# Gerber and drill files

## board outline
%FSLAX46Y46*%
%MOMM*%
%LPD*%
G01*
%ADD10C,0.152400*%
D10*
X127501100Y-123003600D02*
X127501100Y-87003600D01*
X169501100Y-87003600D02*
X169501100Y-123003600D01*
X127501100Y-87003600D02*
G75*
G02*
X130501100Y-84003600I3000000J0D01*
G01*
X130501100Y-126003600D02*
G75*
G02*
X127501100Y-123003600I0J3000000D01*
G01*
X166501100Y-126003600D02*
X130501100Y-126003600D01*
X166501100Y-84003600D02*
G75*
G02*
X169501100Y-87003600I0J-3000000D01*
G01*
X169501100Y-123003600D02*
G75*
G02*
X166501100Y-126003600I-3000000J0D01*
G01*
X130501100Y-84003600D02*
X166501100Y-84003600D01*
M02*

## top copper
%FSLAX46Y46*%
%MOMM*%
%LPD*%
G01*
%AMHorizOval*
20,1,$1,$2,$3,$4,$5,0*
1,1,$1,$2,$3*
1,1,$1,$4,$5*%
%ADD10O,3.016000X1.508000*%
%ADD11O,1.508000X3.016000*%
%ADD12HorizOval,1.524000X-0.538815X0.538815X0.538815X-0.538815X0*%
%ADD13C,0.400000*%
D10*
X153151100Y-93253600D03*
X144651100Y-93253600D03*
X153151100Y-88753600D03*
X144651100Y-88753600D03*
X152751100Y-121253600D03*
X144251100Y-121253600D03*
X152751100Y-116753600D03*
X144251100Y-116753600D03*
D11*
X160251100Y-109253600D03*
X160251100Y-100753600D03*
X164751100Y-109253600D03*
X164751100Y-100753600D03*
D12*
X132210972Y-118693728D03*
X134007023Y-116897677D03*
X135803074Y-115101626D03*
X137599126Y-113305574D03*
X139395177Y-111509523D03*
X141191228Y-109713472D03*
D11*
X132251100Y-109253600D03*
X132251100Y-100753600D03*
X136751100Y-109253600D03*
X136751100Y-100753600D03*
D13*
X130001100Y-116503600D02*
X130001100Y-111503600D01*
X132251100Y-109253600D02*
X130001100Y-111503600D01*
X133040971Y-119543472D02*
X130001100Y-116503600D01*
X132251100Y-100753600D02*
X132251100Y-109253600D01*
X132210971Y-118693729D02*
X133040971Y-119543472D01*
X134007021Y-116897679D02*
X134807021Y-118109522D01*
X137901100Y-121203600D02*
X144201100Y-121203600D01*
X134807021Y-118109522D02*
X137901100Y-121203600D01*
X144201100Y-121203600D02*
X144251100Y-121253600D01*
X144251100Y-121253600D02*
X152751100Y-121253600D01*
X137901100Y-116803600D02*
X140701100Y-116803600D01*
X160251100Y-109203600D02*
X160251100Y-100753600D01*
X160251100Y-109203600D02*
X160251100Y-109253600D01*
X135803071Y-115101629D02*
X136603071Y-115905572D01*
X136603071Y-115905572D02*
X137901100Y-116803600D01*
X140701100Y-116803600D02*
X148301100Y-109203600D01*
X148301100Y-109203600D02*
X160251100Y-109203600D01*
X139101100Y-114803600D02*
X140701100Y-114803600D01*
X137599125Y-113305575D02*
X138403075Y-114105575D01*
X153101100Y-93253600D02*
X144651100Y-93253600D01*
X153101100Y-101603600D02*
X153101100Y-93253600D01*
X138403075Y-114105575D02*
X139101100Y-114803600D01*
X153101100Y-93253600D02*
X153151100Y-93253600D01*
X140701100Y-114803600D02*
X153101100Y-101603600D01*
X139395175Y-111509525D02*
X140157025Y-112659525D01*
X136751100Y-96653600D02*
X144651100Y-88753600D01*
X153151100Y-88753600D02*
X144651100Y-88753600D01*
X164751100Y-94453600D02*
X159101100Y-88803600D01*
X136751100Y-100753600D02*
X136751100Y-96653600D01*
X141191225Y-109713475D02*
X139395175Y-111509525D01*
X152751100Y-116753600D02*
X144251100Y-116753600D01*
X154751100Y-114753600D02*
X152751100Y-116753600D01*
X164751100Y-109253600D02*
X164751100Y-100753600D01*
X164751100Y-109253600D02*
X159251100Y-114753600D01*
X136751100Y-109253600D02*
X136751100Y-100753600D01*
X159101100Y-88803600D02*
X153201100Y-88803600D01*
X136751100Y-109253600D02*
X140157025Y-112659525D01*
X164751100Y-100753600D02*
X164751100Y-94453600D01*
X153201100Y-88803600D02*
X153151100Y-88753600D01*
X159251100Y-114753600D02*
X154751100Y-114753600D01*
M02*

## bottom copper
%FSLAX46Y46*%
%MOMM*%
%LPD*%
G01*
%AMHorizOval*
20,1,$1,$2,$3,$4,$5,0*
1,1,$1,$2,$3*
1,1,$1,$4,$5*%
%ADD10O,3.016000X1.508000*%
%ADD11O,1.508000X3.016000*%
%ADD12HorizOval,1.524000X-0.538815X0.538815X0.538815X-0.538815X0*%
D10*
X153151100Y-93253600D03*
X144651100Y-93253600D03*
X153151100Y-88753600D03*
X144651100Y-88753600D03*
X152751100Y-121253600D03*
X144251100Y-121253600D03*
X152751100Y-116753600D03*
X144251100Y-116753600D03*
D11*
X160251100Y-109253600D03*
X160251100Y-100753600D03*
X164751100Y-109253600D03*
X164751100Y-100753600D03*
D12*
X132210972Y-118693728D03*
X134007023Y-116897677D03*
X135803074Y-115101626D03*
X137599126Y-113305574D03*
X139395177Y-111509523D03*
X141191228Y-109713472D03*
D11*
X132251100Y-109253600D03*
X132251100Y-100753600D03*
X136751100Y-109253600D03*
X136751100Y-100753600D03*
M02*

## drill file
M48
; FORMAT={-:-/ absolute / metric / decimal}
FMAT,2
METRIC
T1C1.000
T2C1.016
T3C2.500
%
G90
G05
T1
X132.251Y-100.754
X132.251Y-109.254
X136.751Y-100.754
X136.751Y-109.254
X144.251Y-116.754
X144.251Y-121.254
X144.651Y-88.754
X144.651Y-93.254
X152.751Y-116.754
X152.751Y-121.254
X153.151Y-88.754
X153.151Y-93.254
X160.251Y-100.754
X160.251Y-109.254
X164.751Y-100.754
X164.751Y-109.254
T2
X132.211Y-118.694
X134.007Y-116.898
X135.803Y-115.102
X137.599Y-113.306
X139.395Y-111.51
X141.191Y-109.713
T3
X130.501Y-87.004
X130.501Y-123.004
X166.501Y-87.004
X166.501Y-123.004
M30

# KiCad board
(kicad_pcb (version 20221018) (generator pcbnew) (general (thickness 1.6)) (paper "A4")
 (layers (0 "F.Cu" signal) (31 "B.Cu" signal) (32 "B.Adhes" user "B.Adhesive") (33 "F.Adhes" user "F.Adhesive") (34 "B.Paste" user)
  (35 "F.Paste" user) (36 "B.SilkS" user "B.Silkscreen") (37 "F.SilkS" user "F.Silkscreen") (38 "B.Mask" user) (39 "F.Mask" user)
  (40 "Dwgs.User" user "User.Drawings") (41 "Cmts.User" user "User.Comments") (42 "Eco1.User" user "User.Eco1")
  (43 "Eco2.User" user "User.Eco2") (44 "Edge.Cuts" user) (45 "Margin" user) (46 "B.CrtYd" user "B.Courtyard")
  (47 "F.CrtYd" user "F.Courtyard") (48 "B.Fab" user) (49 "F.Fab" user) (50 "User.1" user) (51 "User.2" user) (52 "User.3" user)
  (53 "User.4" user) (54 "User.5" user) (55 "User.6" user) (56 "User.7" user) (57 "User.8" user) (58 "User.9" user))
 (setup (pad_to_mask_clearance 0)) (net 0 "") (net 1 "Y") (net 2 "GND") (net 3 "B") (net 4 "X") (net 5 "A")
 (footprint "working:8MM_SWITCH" (layer "F.Cu") (at 148.9011 91.0036 180)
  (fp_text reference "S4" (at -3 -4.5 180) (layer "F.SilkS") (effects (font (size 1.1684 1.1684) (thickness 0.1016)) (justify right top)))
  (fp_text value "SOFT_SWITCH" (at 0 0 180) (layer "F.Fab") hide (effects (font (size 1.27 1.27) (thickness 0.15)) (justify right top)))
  (pad "1" thru_hole oval (at -4.25 -2.25) (size 3.016 1.508) (drill 1) (layers "*.Cu" "*.Mask") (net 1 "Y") (solder_mask_margin 0.1016)
   (thermal_bridge_angle 45))
  (pad "2" thru_hole oval (at 4.25 -2.25 180) (size 3.016 1.508) (drill 1) (layers "*.Cu" "*.Mask") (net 1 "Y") (solder_mask_margin 0.1016)
   (thermal_bridge_angle 45))
  (pad "3" thru_hole oval (at -4.25 2.25 180) (size 3.016 1.508) (drill 1) (layers "*.Cu" "*.Mask") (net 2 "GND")
   (solder_mask_margin 0.1016) (thermal_bridge_angle 45))
  (pad "4" thru_hole oval (at 4.25 2.25 180) (size 3.016 1.508) (drill 1) (layers "*.Cu" "*.Mask") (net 2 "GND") (solder_mask_margin 0.1016)
   (thermal_bridge_angle 45)))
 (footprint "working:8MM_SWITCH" (layer "F.Cu") (at 148.5011 119.0036 180)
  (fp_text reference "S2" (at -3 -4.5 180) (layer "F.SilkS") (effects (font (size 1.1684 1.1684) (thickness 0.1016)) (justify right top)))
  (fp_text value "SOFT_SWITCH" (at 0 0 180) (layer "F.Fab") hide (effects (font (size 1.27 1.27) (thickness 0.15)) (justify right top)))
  (pad "1" thru_hole oval (at -4.25 -2.25) (size 3.016 1.508) (drill 1) (layers "*.Cu" "*.Mask") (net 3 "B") (solder_mask_margin 0.1016)
   (thermal_bridge_angle 45))
  (pad "2" thru_hole oval (at 4.25 -2.25 180) (size 3.016 1.508) (drill 1) (layers "*.Cu" "*.Mask") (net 3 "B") (solder_mask_margin 0.1016)
   (thermal_bridge_angle 45))
  (pad "3" thru_hole oval (at -4.25 2.25 180) (size 3.016 1.508) (drill 1) (layers "*.Cu" "*.Mask") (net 2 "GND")
   (solder_mask_margin 0.1016) (thermal_bridge_angle 45))
  (pad "4" thru_hole oval (at 4.25 2.25 180) (size 3.016 1.508) (drill 1) (layers "*.Cu" "*.Mask") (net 2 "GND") (solder_mask_margin 0.1016)
   (thermal_bridge_angle 45)))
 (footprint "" (layer "F.Cu") (at 166.5011 123.0036)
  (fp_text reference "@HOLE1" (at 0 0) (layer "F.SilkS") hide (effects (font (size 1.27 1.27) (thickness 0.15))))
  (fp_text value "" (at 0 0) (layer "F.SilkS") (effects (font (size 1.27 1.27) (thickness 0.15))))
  (pad "" np_thru_hole circle (at 0 0) (size 2.5 2.5) (drill 2.5) (layers "*.Cu" "*.Mask")))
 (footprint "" (layer "F.Cu") (at 166.5011 87.0036)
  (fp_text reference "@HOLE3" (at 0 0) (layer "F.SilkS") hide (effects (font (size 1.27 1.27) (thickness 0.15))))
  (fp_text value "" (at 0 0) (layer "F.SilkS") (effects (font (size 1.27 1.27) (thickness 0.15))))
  (pad "" np_thru_hole circle (at 0 0) (size 2.5 2.5) (drill 2.5) (layers "*.Cu" "*.Mask")))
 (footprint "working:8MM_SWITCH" (layer "F.Cu") (at 162.5011 105.0036 90)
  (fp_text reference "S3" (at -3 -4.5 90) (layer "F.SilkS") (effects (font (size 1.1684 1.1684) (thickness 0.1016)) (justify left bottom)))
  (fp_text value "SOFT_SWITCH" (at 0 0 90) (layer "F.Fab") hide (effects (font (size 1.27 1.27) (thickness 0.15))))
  (pad "1" thru_hole oval (at -4.25 -2.25 270) (size 3.016 1.508) (drill 1) (layers "*.Cu" "*.Mask") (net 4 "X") (solder_mask_margin 0.1016)
   (thermal_bridge_angle 45))
  (pad "2" thru_hole oval (at 4.25 -2.25 90) (size 3.016 1.508) (drill 1) (layers "*.Cu" "*.Mask") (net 4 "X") (solder_mask_margin 0.1016)
   (thermal_bridge_angle 45))
  (pad "3" thru_hole oval (at -4.25 2.25 90) (size 3.016 1.508) (drill 1) (layers "*.Cu" "*.Mask") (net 2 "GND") (solder_mask_margin 0.1016)
   (thermal_bridge_angle 45))
  (pad "4" thru_hole oval (at 4.25 2.25 90) (size 3.016 1.508) (drill 1) (layers "*.Cu" "*.Mask") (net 2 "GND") (solder_mask_margin 0.1016)
   (thermal_bridge_angle 45)))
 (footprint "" (layer "F.Cu") (at 130.5011 123.0036)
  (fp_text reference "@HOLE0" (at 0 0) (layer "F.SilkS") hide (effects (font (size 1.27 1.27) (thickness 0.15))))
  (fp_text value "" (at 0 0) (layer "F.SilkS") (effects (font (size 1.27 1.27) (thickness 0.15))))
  (pad "" np_thru_hole circle (at 0 0) (size 2.5 2.5) (drill 2.5) (layers "*.Cu" "*.Mask")))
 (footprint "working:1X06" (layer "F.Cu") (at 136.7011 114.2036 45)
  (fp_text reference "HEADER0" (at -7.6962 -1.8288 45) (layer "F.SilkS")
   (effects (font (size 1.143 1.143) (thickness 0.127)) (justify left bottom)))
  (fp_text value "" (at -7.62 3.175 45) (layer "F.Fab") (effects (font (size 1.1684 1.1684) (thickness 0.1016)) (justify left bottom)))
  (pad "1" thru_hole oval (at -6.35 0 135) (size 3.048 1.524) (drill 1.016) (layers "*.Cu" "*.Mask") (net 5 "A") (solder_mask_margin 0.1016)
   (thermal_bridge_angle 45))
  (pad "2" thru_hole oval (at -3.81 0 135) (size 3.048 1.524) (drill 1.016) (layers "*.Cu" "*.Mask") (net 3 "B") (solder_mask_margin 0.1016)
   (thermal_bridge_angle 45))
  (pad "3" thru_hole oval (at -1.27 0 135) (size 3.048 1.524) (drill 1.016) (layers "*.Cu" "*.Mask") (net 4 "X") (solder_mask_margin 0.1016)
   (thermal_bridge_angle 45))
  (pad "4" thru_hole oval (at 1.27 0 135) (size 3.048 1.524) (drill 1.016) (layers "*.Cu" "*.Mask") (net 1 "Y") (solder_mask_margin 0.1016)
   (thermal_bridge_angle 45))
  (pad "5" thru_hole oval (at 3.81 0 135) (size 3.048 1.524) (drill 1.016) (layers "*.Cu" "*.Mask") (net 2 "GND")
   (solder_mask_margin 0.1016) (thermal_bridge_angle 45))
  (pad "6" thru_hole oval (at 6.35 0 135) (size 3.048 1.524) (drill 1.016) (layers "*.Cu" "*.Mask") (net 2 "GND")
   (solder_mask_margin 0.1016) (thermal_bridge_angle 45)))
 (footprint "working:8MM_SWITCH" (layer "F.Cu") (at 134.5011 105.0036 90)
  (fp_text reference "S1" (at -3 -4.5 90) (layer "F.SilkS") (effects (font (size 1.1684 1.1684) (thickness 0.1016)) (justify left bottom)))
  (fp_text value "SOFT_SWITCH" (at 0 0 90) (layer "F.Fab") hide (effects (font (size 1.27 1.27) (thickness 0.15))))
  (pad "1" thru_hole oval (at -4.25 -2.25 270) (size 3.016 1.508) (drill 1) (layers "*.Cu" "*.Mask") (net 5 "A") (solder_mask_margin 0.1016)
   (thermal_bridge_angle 45))
  (pad "2" thru_hole oval (at 4.25 -2.25 90) (size 3.016 1.508) (drill 1) (layers "*.Cu" "*.Mask") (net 5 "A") (solder_mask_margin 0.1016)
   (thermal_bridge_angle 45))
  (pad "3" thru_hole oval (at -4.25 2.25 90) (size 3.016 1.508) (drill 1) (layers "*.Cu" "*.Mask") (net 2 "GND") (solder_mask_margin 0.1016)
   (thermal_bridge_angle 45))
  (pad "4" thru_hole oval (at 4.25 2.25 90) (size 3.016 1.508) (drill 1) (layers "*.Cu" "*.Mask") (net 2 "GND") (solder_mask_margin 0.1016)
   (thermal_bridge_angle 45)))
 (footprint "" (layer "F.Cu") (at 130.5011 87.0036)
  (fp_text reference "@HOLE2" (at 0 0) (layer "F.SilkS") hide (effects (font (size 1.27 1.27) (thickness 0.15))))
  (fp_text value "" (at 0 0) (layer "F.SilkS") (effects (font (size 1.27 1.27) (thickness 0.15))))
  (pad "" np_thru_hole circle (at 0 0) (size 2.5 2.5) (drill 2.5) (layers "*.Cu" "*.Mask")))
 (gr_line (start 127.5011 123.0036) (end 127.5011 87.0036) (stroke (width 0.1524) (type solid)) (layer "Edge.Cuts"))
 (gr_line (start 169.5011 87.0036) (end 169.5011 123.0036) (stroke (width 0.1524) (type solid)) (layer "Edge.Cuts"))
 (gr_arc (start 127.5011 87.0036) (mid 128.37978 84.88228) (end 130.5011 84.0036) (stroke (width 0.1524) (type solid)) (layer "Edge.Cuts"))
 (gr_arc (start 130.5011 126.0036) (mid 128.37978 125.12492) (end 127.5011 123.0036) (stroke (width 0.1524) (type solid))
  (layer "Edge.Cuts"))
 (gr_line (start 166.5011 126.0036) (end 130.5011 126.0036) (stroke (width 0.1524) (type solid)) (layer "Edge.Cuts"))
 (gr_arc (start 166.5011 84.0036) (mid 168.62242 84.88228) (end 169.5011 87.0036) (stroke (width 0.1524) (type solid)) (layer "Edge.Cuts"))
 (gr_arc (start 169.5011 123.0036) (mid 168.62242 125.12492) (end 166.5011 126.0036) (stroke (width 0.1524) (type solid))
  (layer "Edge.Cuts"))
 (gr_line (start 130.5011 84.0036) (end 166.5011 84.0036) (stroke (width 0.1524) (type solid)) (layer "Edge.Cuts"))
 (segment (start 130.0011 116.5036) (end 130.0011 111.5036) (width 0.4) (layer "F.Cu") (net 5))
 (segment (start 132.2511 109.2536) (end 130.0011 111.5036) (width 0.4) (layer "F.Cu") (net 5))
 (segment (start 133.040971 119.543472) (end 130.0011 116.5036) (width 0.4) (layer "F.Cu") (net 5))
 (segment (start 132.2511 100.7536) (end 132.2511 109.2536) (width 0.4) (layer "F.Cu") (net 5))
 (segment (start 132.210971 118.693729) (end 133.040971 119.543472) (width 0.4) (layer "F.Cu") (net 5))
 (segment (start 134.007021 116.897679) (end 134.807021 118.109522) (width 0.4) (layer "F.Cu") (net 3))
 (segment (start 137.9011 121.2036) (end 144.2011 121.2036) (width 0.4) (layer "F.Cu") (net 3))
 (segment (start 134.807021 118.109522) (end 137.9011 121.2036) (width 0.4) (layer "F.Cu") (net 3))
 (segment (start 144.2011 121.2036) (end 144.2511 121.2536) (width 0.4) (layer "F.Cu") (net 3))
 (segment (start 144.2511 121.2536) (end 152.7511 121.2536) (width 0.4) (layer "F.Cu") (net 3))
 (segment (start 137.9011 116.8036) (end 140.7011 116.8036) (width 0.4) (layer "F.Cu") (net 4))
 (segment (start 160.2511 109.2036) (end 160.2511 100.7536) (width 0.4) (layer "F.Cu") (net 4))
 (segment (start 160.2511 109.2036) (end 160.2511 109.2536) (width 0.4) (layer "F.Cu") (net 4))
 (segment (start 135.803071 115.101629) (end 136.603071 115.905572) (width 0.4) (layer "F.Cu") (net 4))
 (segment (start 136.603071 115.905572) (end 137.9011 116.8036) (width 0.4) (layer "F.Cu") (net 4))
 (segment (start 140.7011 116.8036) (end 148.3011 109.2036) (width 0.4) (layer "F.Cu") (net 4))
 (segment (start 148.3011 109.2036) (end 160.2511 109.2036) (width 0.4) (layer "F.Cu") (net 4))
 (segment (start 139.1011 114.8036) (end 140.7011 114.8036) (width 0.4) (layer "F.Cu") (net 1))
 (segment (start 137.599125 113.305575) (end 138.403075 114.105575) (width 0.4) (layer "F.Cu") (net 1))
 (segment (start 153.1011 93.2536) (end 144.6511 93.2536) (width 0.4) (layer "F.Cu") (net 1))
 (segment (start 153.1011 101.6036) (end 153.1011 93.2536) (width 0.4) (layer "F.Cu") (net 1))
 (segment (start 138.403075 114.105575) (end 139.1011 114.8036) (width 0.4) (layer "F.Cu") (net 1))
 (segment (start 153.1011 93.2536) (end 153.1511 93.2536) (width 0.4) (layer "F.Cu") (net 1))
 (segment (start 140.7011 114.8036) (end 153.1011 101.6036) (width 0.4) (layer "F.Cu") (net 1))
 (segment (start 139.395175 111.509525) (end 140.157025 112.659525) (width 0.4) (layer "F.Cu") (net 2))
 (segment (start 136.7511 96.6536) (end 144.6511 88.7536) (width 0.4) (layer "F.Cu") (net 2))
 (segment (start 153.1511 88.7536) (end 144.6511 88.7536) (width 0.4) (layer "F.Cu") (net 2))
 (segment (start 164.7511 94.4536) (end 159.1011 88.8036) (width 0.4) (layer "F.Cu") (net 2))
 (segment (start 136.7511 100.7536) (end 136.7511 96.6536) (width 0.4) (layer "F.Cu") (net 2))
 (segment (start 141.191225 109.713475) (end 139.395175 111.509525) (width 0.4) (layer "F.Cu") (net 2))
 (segment (start 152.7511 116.7536) (end 144.2511 116.7536) (width 0.4) (layer "F.Cu") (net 2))
 (segment (start 154.7511 114.7536) (end 152.7511 116.7536) (width 0.4) (layer "F.Cu") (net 2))
 (segment (start 164.7511 109.2536) (end 164.7511 100.7536) (width 0.4) (layer "F.Cu") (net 2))
 (segment (start 164.7511 109.2536) (end 159.2511 114.7536) (width 0.4) (layer "F.Cu") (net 2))
 (segment (start 136.7511 109.2536) (end 136.7511 100.7536) (width 0.4) (layer "F.Cu") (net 2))
 (segment (start 159.1011 88.8036) (end 153.2011 88.8036) (width 0.4) (layer "F.Cu") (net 2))
 (segment (start 136.7511 109.2536) (end 140.157025 112.659525) (width 0.4) (layer "F.Cu") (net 2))
 (segment (start 164.7511 100.7536) (end 164.7511 94.4536) (width 0.4) (layer "F.Cu") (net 2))
 (segment (start 153.2011 88.8036) (end 153.1511 88.7536) (width 0.4) (layer "F.Cu") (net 2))
 (segment (start 159.2511 114.7536) (end 154.7511 114.7536) (width 0.4) (layer "F.Cu") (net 2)))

